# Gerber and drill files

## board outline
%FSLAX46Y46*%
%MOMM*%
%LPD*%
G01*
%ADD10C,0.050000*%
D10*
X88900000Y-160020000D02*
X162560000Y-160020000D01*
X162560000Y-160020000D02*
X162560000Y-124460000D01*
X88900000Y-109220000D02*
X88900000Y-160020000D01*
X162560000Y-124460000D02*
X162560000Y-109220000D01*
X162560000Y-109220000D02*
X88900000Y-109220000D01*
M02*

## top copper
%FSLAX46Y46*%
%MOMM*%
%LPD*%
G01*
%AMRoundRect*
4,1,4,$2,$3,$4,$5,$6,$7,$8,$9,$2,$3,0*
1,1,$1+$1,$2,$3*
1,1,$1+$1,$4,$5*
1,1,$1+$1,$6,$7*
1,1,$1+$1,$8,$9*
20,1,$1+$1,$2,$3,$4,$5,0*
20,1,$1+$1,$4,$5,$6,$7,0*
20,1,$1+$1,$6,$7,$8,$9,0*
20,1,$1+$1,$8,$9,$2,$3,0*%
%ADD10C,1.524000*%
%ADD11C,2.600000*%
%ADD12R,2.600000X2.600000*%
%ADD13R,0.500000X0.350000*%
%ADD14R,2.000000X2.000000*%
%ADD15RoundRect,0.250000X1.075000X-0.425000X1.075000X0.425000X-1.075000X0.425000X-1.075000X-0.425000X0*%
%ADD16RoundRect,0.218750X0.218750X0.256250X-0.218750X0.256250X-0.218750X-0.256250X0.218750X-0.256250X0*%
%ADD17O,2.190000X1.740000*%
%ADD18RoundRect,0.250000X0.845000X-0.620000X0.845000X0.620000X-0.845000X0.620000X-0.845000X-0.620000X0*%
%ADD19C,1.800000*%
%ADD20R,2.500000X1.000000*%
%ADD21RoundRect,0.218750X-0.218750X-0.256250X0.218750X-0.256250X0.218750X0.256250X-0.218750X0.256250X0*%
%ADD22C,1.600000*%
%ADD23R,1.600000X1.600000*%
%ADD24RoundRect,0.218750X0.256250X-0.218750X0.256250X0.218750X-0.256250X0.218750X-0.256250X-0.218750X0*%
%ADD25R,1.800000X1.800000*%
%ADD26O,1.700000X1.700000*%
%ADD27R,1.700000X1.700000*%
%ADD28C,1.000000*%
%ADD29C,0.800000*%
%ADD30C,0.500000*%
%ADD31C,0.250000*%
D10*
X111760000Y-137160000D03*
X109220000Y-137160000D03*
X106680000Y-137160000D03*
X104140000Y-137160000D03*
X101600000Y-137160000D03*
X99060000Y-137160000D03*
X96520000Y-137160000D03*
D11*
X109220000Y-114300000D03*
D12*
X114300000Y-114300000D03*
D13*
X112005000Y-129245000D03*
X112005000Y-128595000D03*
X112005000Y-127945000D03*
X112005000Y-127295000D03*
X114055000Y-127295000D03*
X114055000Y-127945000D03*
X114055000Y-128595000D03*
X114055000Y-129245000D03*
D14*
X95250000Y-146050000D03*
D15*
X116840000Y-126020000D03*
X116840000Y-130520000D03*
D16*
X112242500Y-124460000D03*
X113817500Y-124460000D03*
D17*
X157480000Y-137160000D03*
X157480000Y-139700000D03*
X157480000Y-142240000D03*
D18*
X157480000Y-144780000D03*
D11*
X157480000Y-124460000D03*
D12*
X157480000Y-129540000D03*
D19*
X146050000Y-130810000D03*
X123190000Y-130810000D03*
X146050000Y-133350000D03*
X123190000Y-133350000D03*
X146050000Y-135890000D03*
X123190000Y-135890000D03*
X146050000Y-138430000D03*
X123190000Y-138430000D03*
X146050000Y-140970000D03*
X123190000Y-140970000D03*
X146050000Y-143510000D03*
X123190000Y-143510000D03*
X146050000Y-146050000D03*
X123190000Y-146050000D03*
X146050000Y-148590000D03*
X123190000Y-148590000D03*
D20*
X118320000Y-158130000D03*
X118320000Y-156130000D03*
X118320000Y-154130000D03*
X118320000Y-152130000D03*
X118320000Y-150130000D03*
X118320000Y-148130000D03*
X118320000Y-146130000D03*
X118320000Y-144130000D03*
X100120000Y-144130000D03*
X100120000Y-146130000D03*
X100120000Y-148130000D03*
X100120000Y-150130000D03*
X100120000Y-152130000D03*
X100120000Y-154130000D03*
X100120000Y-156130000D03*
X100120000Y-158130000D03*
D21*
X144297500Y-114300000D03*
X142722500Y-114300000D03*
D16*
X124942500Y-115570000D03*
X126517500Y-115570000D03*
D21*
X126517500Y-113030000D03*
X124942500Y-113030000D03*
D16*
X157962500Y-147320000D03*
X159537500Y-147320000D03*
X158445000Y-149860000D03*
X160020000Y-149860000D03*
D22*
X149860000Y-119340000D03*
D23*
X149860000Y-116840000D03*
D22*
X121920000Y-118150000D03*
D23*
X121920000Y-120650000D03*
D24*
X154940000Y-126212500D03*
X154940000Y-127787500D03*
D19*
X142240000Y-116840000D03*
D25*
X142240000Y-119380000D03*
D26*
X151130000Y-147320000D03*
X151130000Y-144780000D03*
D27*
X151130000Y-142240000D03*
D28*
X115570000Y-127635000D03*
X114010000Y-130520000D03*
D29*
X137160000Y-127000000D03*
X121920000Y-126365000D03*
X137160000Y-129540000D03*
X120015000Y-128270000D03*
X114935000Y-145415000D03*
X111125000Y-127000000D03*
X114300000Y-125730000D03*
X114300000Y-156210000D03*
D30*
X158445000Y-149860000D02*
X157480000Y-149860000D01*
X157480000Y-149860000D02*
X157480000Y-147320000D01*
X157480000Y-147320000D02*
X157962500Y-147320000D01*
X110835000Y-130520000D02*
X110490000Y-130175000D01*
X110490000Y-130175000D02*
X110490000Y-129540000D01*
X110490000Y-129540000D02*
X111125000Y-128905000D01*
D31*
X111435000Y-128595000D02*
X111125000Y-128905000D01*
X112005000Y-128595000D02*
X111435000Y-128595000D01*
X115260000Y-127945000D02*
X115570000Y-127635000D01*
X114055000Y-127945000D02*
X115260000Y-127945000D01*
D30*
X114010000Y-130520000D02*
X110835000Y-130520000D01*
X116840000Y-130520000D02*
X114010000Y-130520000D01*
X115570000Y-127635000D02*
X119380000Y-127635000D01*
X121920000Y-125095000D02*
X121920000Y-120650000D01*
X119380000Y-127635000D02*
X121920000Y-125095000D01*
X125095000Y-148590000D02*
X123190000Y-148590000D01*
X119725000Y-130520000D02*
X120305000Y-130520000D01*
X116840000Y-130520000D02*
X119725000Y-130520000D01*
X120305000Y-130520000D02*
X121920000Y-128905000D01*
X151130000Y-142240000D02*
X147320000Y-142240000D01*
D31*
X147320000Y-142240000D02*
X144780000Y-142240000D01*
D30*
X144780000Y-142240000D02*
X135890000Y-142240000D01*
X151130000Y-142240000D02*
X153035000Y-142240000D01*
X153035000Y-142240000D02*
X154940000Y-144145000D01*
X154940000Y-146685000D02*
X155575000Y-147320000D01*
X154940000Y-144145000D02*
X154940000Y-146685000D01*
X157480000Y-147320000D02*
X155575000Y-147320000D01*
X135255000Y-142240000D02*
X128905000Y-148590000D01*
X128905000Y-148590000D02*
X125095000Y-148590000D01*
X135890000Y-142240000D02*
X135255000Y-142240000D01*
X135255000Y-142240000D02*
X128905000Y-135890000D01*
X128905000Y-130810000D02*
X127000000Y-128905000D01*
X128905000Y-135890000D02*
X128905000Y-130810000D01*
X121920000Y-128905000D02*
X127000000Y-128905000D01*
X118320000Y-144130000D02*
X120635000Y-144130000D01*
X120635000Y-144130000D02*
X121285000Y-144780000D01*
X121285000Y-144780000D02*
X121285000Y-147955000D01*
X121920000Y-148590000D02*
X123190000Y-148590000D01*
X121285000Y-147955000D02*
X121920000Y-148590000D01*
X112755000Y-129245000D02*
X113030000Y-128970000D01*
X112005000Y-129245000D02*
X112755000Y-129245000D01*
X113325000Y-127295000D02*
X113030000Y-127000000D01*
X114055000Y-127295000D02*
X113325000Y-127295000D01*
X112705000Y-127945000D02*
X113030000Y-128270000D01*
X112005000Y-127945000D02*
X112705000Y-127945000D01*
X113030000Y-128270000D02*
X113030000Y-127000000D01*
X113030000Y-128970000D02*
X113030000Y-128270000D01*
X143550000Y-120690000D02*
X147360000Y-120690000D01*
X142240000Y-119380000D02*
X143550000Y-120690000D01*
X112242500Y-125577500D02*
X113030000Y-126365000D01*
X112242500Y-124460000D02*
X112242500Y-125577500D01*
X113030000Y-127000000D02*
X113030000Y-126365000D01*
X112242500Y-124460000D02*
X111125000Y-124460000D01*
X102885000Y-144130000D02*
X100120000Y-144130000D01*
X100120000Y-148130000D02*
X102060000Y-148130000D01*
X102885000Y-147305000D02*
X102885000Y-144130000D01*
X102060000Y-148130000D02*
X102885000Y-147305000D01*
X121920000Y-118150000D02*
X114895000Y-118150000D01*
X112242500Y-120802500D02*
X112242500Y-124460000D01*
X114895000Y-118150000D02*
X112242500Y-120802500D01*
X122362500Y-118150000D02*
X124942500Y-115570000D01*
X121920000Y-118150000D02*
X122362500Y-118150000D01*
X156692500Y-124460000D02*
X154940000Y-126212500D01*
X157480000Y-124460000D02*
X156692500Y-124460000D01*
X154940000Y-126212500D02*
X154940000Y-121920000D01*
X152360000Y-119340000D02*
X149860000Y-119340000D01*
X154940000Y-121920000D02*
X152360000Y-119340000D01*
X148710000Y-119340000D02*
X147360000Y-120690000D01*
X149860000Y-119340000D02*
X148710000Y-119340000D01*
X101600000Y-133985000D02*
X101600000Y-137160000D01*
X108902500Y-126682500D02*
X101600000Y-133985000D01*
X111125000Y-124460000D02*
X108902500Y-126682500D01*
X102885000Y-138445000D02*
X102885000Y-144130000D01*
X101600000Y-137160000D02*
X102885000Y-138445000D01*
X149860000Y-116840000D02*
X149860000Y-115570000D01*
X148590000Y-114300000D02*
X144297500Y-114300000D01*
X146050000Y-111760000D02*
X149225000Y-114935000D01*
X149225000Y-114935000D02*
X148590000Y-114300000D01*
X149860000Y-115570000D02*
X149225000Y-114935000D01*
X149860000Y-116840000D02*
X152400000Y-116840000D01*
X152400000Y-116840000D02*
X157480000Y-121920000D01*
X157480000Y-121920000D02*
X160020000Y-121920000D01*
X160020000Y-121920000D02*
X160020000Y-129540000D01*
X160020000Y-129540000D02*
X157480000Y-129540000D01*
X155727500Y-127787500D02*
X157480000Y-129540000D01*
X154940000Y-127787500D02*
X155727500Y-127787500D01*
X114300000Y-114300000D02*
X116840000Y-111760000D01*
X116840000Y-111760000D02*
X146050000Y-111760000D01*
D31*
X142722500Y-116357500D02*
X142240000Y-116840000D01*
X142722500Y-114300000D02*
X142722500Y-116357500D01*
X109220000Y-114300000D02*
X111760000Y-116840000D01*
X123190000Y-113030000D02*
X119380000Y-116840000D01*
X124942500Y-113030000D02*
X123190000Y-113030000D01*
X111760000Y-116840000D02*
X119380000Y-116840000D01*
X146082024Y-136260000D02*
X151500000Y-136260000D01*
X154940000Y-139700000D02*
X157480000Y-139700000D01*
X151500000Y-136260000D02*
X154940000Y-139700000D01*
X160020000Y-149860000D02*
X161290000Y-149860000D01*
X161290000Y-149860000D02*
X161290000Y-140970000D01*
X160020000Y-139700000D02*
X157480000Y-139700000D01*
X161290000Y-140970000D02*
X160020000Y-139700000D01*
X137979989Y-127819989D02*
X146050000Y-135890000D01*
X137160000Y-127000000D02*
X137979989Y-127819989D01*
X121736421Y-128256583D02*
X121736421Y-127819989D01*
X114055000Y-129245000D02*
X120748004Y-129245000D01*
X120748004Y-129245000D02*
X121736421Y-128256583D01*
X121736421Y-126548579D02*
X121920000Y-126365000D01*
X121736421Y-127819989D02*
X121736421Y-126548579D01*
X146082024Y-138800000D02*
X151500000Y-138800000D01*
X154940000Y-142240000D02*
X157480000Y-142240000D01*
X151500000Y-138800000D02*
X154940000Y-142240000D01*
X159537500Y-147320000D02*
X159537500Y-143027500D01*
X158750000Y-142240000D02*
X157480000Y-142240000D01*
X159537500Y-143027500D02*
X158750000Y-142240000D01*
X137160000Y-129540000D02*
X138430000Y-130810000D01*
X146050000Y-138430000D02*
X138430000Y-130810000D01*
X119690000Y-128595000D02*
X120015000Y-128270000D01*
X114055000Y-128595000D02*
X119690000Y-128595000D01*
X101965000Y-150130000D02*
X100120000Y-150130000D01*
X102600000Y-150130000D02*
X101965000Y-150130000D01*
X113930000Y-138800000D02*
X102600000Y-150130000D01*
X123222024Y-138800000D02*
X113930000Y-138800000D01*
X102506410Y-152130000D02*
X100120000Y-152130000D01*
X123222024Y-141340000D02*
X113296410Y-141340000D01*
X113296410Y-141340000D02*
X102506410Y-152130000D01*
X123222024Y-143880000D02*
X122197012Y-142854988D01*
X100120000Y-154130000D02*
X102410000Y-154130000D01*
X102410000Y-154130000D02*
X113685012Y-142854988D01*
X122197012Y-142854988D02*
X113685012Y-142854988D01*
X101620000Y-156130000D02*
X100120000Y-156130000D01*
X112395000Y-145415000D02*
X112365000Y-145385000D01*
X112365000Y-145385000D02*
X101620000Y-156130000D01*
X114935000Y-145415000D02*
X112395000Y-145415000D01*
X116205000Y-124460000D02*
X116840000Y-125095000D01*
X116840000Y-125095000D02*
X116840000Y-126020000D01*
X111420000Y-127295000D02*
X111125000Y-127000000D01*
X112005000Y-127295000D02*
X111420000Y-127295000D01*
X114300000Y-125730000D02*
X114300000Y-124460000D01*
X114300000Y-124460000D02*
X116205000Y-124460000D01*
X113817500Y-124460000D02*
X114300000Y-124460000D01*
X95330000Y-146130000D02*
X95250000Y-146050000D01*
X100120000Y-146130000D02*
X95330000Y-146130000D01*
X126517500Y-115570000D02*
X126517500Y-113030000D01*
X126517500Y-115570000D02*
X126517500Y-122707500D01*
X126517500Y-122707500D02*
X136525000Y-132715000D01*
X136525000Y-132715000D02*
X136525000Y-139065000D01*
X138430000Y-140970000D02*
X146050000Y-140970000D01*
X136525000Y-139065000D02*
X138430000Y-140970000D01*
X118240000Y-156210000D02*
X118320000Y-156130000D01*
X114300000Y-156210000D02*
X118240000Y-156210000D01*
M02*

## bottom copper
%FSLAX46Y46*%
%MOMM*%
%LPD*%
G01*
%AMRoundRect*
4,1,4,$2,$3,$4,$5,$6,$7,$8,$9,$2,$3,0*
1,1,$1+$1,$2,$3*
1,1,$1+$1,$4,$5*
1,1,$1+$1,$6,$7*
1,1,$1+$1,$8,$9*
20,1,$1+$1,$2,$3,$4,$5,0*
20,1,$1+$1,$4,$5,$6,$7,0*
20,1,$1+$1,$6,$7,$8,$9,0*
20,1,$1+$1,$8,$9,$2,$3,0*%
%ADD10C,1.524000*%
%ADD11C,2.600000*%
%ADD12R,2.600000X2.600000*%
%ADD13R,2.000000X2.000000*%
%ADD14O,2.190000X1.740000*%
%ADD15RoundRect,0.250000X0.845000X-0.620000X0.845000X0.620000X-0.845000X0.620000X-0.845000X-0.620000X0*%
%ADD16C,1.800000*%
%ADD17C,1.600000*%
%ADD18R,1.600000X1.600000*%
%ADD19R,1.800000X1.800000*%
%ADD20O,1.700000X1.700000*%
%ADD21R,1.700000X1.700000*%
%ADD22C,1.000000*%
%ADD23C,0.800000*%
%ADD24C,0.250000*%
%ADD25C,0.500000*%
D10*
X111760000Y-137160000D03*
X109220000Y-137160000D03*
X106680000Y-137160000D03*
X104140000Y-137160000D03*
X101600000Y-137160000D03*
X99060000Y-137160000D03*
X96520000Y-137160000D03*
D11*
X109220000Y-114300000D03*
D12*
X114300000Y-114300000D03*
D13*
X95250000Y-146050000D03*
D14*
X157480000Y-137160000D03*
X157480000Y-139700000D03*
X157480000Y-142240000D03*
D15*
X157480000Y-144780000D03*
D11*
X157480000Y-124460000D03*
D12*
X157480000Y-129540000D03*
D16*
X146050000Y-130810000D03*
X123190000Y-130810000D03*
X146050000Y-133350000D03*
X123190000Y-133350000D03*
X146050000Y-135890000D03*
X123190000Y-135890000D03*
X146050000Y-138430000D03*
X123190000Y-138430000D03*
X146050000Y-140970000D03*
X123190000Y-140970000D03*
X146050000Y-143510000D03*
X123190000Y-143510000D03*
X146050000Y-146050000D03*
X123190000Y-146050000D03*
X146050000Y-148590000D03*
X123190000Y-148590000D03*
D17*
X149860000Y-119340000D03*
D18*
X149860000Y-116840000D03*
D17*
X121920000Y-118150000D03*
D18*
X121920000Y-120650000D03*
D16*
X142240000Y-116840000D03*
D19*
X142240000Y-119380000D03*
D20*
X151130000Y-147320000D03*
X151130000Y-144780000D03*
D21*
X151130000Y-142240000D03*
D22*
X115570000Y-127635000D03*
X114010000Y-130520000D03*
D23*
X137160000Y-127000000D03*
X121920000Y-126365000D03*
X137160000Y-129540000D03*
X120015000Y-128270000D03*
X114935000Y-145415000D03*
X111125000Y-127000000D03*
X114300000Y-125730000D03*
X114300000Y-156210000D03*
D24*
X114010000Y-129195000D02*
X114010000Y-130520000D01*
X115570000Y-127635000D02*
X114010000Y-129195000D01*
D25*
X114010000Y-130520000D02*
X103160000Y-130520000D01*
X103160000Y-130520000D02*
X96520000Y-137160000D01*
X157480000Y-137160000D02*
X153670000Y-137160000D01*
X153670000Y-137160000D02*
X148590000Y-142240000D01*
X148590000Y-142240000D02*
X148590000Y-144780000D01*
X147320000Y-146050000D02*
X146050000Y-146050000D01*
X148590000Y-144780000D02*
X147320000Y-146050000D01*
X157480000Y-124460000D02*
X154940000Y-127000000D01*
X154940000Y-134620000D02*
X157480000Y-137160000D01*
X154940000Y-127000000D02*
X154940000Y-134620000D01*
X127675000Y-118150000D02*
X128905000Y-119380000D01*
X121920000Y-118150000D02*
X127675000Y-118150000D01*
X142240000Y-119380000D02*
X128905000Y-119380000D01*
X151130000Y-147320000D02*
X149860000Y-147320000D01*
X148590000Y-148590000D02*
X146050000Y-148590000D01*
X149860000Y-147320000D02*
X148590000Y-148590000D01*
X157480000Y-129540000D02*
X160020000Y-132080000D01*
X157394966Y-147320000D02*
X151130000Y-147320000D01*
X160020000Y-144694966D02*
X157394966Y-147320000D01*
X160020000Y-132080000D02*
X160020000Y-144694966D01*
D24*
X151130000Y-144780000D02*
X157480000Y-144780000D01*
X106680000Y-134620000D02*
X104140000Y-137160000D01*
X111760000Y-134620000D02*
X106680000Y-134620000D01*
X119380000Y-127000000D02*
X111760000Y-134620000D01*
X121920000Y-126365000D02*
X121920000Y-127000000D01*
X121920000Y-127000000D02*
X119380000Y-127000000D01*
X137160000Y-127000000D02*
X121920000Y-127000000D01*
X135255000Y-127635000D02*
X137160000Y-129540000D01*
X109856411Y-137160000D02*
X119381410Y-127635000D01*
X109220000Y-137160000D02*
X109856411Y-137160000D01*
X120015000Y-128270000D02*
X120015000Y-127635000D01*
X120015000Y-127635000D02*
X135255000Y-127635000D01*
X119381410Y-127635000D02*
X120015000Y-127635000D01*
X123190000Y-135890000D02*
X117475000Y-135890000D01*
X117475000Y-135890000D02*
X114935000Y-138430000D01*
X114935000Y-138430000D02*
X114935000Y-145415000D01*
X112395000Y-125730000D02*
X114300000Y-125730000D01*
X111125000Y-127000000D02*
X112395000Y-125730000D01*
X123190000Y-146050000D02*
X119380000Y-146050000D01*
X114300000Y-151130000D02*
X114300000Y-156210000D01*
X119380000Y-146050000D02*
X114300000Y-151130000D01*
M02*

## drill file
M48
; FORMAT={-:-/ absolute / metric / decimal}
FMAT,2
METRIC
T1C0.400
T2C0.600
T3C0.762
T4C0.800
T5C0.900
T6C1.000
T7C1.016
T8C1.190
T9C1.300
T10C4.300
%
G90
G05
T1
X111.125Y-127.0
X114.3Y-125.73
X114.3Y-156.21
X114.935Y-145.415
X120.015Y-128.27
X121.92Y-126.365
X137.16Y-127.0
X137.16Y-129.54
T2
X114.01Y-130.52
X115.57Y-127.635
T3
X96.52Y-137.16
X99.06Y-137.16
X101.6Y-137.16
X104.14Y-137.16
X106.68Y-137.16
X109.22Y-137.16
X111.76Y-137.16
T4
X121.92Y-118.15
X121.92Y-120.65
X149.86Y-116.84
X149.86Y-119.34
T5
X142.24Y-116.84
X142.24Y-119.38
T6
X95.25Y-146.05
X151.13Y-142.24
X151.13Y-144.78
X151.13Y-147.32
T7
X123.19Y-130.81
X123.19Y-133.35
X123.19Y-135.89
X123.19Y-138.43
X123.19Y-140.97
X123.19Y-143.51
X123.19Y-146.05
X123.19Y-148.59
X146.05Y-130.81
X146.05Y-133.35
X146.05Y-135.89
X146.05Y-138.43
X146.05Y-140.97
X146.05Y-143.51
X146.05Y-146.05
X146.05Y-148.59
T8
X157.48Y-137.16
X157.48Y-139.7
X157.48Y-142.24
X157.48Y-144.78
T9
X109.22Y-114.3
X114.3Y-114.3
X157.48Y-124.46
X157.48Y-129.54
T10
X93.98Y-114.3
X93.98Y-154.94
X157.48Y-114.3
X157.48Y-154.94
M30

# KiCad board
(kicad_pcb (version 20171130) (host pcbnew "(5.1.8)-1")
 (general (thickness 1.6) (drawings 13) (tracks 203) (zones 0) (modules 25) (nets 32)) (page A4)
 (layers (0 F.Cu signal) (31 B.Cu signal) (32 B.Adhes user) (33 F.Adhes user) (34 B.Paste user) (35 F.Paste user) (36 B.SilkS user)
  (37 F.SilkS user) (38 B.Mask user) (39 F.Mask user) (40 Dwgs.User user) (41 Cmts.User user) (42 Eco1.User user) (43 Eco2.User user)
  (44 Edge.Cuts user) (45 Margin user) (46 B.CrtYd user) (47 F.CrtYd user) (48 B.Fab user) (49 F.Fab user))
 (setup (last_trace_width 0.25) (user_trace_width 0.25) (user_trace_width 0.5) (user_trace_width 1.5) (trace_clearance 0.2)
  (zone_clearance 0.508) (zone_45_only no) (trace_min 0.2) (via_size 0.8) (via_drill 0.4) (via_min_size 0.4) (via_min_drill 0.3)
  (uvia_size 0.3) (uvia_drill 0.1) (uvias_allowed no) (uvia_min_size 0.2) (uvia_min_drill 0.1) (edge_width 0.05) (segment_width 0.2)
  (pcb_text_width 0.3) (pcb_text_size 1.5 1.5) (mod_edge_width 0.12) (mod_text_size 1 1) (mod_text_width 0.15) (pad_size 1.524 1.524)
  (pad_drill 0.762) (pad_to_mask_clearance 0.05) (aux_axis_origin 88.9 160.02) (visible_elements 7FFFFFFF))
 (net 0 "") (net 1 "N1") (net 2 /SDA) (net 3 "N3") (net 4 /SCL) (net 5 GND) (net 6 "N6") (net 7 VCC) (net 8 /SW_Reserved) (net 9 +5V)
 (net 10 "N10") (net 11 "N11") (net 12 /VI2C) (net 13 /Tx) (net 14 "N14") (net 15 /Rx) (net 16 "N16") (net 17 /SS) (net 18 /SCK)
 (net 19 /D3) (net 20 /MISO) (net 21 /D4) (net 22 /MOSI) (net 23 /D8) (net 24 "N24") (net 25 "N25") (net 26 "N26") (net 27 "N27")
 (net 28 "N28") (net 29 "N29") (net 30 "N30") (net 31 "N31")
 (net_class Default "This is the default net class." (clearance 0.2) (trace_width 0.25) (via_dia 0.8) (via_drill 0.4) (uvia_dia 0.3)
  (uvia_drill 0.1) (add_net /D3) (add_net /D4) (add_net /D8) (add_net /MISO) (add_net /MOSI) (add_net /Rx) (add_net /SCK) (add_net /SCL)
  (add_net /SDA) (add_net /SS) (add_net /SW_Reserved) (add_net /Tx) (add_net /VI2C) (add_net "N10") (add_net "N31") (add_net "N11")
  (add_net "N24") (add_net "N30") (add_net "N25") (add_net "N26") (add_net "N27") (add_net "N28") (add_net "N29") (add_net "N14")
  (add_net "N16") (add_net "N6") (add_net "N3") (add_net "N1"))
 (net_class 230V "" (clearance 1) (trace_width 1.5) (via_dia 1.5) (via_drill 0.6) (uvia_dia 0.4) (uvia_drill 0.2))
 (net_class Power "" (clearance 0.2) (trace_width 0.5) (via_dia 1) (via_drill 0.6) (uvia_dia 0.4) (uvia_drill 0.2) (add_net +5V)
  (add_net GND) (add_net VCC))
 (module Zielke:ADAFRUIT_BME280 (layer F.Cu) (at 104.14 137.16 90)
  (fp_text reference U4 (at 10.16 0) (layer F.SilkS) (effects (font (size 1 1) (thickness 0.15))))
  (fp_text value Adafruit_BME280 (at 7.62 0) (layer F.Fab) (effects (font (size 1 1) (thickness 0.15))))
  (pad 7 thru_hole circle (at 0 7.62 90) (size 1.524 1.524) (drill 0.762) (layers *.Cu *.Mask) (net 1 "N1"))
  (pad 6 thru_hole circle (at 0 5.08 90) (size 1.524 1.524) (drill 0.762) (layers *.Cu *.Mask) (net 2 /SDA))
  (pad 5 thru_hole circle (at 0 2.54 90) (size 1.524 1.524) (drill 0.762) (layers *.Cu *.Mask) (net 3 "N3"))
  (pad 4 thru_hole circle (at 0 0 90) (size 1.524 1.524) (drill 0.762) (layers *.Cu *.Mask) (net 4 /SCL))
  (pad 3 thru_hole circle (at 0 -2.54 90) (size 1.524 1.524) (drill 0.762) (layers *.Cu *.Mask) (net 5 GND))
  (pad 2 thru_hole circle (at 0 -5.08 90) (size 1.524 1.524) (drill 0.762) (layers *.Cu *.Mask) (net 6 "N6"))
  (pad 1 thru_hole circle (at 0 -7.62 90) (size 1.524 1.524) (drill 0.762) (layers *.Cu *.Mask) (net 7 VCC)))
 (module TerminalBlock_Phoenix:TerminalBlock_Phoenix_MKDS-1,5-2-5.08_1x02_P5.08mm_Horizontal (layer F.Cu) (at 114.3 114.3 180)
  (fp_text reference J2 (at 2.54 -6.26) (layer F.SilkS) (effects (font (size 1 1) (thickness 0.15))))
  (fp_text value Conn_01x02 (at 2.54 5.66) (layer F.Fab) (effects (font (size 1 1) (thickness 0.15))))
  (pad 2 thru_hole circle (at 5.08 0 180) (size 2.6 2.6) (drill 1.3) (layers *.Cu *.Mask) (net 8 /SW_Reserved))
  (pad 1 thru_hole rect (at 0 0 180) (size 2.6 2.6) (drill 1.3) (layers *.Cu *.Mask) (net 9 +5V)))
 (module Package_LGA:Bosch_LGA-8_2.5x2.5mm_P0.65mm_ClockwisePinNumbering (layer F.Cu) (at 113.03 128.27 270)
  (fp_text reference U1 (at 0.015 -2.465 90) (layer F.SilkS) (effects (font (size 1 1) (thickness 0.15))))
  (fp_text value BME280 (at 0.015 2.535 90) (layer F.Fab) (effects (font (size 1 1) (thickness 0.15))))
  (pad 5 smd rect (at 0.975 1.025) (size 0.5 0.35) (layers F.Cu F.Paste F.Mask) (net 5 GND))
  (pad 6 smd rect (at 0.325 1.025) (size 0.5 0.35) (layers F.Cu F.Paste F.Mask) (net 7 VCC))
  (pad 7 smd rect (at -0.325 1.025) (size 0.5 0.35) (layers F.Cu F.Paste F.Mask) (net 5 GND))
  (pad 8 smd rect (at -0.975 1.025) (size 0.5 0.35) (layers F.Cu F.Paste F.Mask) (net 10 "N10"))
  (pad 1 smd rect (at -0.975 -1.025) (size 0.5 0.35) (layers F.Cu F.Paste F.Mask) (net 5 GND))
  (pad 2 smd rect (at -0.325 -1.025) (size 0.5 0.35) (layers F.Cu F.Paste F.Mask) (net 7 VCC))
  (pad 3 smd rect (at 0.325 -1.025) (size 0.5 0.35) (layers F.Cu F.Paste F.Mask) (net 2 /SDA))
  (pad 4 smd rect (at 0.975 -1.025) (size 0.5 0.35) (layers F.Cu F.Paste F.Mask) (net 4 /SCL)))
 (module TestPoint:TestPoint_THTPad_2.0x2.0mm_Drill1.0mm (layer F.Cu) (at 95.25 146.05)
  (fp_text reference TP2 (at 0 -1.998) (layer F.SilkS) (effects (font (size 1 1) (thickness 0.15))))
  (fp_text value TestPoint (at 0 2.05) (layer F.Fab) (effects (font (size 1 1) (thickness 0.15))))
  (pad 1 thru_hole rect (at 0 0) (size 2 2) (drill 1) (layers *.Cu *.Mask) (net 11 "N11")))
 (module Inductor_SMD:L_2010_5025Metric (layer F.Cu) (at 116.84 128.27 90)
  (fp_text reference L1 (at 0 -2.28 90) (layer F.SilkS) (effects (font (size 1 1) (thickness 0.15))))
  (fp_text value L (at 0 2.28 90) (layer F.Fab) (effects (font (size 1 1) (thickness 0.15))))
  (pad 2 smd roundrect (at 2.25 0 90) (size 1.35 2.65) (layers F.Cu F.Paste F.Mask) (roundrect_rratio 0.185185) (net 10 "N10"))
  (pad 1 smd roundrect (at -2.25 0 90) (size 1.35 2.65) (layers F.Cu F.Paste F.Mask) (roundrect_rratio 0.185185) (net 7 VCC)))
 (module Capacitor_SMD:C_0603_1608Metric (layer F.Cu) (at 113.03 124.46 180)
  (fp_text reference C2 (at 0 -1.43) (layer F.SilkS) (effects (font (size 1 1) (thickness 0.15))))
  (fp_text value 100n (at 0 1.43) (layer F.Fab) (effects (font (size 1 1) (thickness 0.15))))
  (pad 2 smd roundrect (at 0.7875 0 180) (size 0.875 0.95) (layers F.Cu F.Paste F.Mask) (roundrect_rratio 0.25) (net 5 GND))
  (pad 1 smd roundrect (at -0.7875 0 180) (size 0.875 0.95) (layers F.Cu F.Paste F.Mask) (roundrect_rratio 0.25) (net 10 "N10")))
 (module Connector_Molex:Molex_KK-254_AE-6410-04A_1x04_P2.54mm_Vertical (layer F.Cu) (at 157.48 144.78 90)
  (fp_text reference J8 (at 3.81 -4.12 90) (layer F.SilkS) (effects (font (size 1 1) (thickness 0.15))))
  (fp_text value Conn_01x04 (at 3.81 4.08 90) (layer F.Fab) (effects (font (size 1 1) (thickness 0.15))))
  (pad 4 thru_hole oval (at 7.62 0 90) (size 1.74 2.19) (drill 1.19) (layers *.Cu *.Mask) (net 5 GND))
  (pad 3 thru_hole oval (at 5.08 0 90) (size 1.74 2.19) (drill 1.19) (layers *.Cu *.Mask) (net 4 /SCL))
  (pad 2 thru_hole oval (at 2.54 0 90) (size 1.74 2.19) (drill 1.19) (layers *.Cu *.Mask) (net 2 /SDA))
  (pad 1 thru_hole roundrect (at 0 0 90) (size 1.74 2.19) (drill 1.19) (layers *.Cu *.Mask) (roundrect_rratio 0.143678) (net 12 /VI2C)))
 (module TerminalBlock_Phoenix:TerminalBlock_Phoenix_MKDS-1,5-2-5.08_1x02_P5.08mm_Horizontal (layer F.Cu) (at 157.48 129.54 90)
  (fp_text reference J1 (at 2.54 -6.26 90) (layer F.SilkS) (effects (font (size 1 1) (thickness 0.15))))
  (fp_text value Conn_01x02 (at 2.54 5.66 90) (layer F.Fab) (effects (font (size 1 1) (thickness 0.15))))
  (pad 2 thru_hole circle (at 5.08 0 90) (size 2.6 2.6) (drill 1.3) (layers *.Cu *.Mask) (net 5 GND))
  (pad 1 thru_hole rect (at 0 0 90) (size 2.6 2.6) (drill 1.3) (layers *.Cu *.Mask) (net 9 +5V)))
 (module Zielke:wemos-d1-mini (layer F.Cu) (at 134.62 139.7 90)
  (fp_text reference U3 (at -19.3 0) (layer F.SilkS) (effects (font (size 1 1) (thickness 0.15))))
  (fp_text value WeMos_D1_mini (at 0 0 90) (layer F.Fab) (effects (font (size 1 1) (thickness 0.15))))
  (pad 16 thru_hole circle (at 8.89 11.43 90) (size 1.8 1.8) (drill 1.016) (layers *.Cu *.Mask) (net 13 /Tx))
  (pad 1 thru_hole circle (at 8.89 -11.43 90) (size 1.8 1.8) (drill 1.016) (layers *.Cu *.Mask) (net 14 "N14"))
  (pad 15 thru_hole circle (at 6.35 11.43 90) (size 1.8 1.8) (drill 1.016) (layers *.Cu *.Mask) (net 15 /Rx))
  (pad 2 thru_hole circle (at 6.35 -11.43 90) (size 1.8 1.8) (drill 1.016) (layers *.Cu *.Mask) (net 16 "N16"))
  (pad 14 thru_hole circle (at 3.81 11.43 90) (size 1.8 1.8) (drill 1.016) (layers *.Cu *.Mask) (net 4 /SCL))
  (pad 3 thru_hole circle (at 3.81 -11.43 90) (size 1.8 1.8) (drill 1.016) (layers *.Cu *.Mask) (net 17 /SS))
  (pad 13 thru_hole circle (at 1.27 11.43 90) (size 1.8 1.8) (drill 1.016) (layers *.Cu *.Mask) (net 2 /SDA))
  (pad 4 thru_hole circle (at 1.27 -11.43 90) (size 1.8 1.8) (drill 1.016) (layers *.Cu *.Mask) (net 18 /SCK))
  (pad 12 thru_hole circle (at -1.27 11.43 90) (size 1.8 1.8) (drill 1.016) (layers *.Cu *.Mask) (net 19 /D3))
  (pad 5 thru_hole circle (at -1.27 -11.43 90) (size 1.8 1.8) (drill 1.016) (layers *.Cu *.Mask) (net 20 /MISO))
  (pad 11 thru_hole circle (at -3.81 11.43 90) (size 1.8 1.8) (drill 1.016) (layers *.Cu *.Mask) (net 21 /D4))
  (pad 6 thru_hole circle (at -3.81 -11.43 180) (size 1.8 1.8) (drill 1.016) (layers *.Cu *.Mask) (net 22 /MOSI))
  (pad 10 thru_hole circle (at -6.35 11.43 90) (size 1.8 1.8) (drill 1.016) (layers *.Cu *.Mask) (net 5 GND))
  (pad 7 thru_hole circle (at -6.35 -11.43 90) (size 1.8 1.8) (drill 1.016) (layers *.Cu *.Mask) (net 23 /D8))
  (pad 9 thru_hole circle (at -8.89 11.43 90) (size 1.8 1.8) (drill 1.016) (layers *.Cu *.Mask) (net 9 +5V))
  (pad 8 thru_hole circle (at -8.89 -11.43 90) (size 1.8 1.8) (drill 1.016) (layers *.Cu *.Mask) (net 7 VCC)))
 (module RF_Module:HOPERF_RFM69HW (layer F.Cu) (at 109.22 151.13 180)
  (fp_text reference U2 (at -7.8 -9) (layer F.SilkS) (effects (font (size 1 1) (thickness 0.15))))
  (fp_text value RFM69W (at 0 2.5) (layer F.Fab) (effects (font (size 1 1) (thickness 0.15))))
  (pad 1 smd rect (at -9.1 -7 180) (size 2.5 1) (layers F.Cu F.Paste F.Mask) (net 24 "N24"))
  (pad 2 smd rect (at -9.1 -5 180) (size 2.5 1) (layers F.Cu F.Paste F.Mask) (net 23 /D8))
  (pad 3 smd rect (at -9.1 -3 180) (size 2.5 1) (layers F.Cu F.Paste F.Mask) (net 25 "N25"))
  (pad 4 smd rect (at -9.1 -1 180) (size 2.5 1) (layers F.Cu F.Paste F.Mask) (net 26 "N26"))
  (pad 5 smd rect (at -9.1 1 180) (size 2.5 1) (layers F.Cu F.Paste F.Mask) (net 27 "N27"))
  (pad 6 smd rect (at -9.1 3 180) (size 2.5 1) (layers F.Cu F.Paste F.Mask) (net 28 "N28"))
  (pad 7 smd rect (at -9.1 5 180) (size 2.5 1) (layers F.Cu F.Paste F.Mask) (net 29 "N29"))
  (pad 8 smd rect (at -9.1 7 180) (size 2.5 1) (layers F.Cu F.Paste F.Mask) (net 7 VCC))
  (pad 9 smd rect (at 9.1 7 180) (size 2.5 1) (layers F.Cu F.Paste F.Mask) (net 5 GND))
  (pad 10 smd rect (at 9.1 5 180) (size 2.5 1) (layers F.Cu F.Paste F.Mask) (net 11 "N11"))
  (pad 11 smd rect (at 9.1 3 180) (size 2.5 1) (layers F.Cu F.Paste F.Mask) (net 5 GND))
  (pad 12 smd rect (at 9.1 1 180) (size 2.5 1) (layers F.Cu F.Paste F.Mask) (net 18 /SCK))
  (pad 13 smd rect (at 9.1 -1 180) (size 2.5 1) (layers F.Cu F.Paste F.Mask) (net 20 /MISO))
  (pad 14 smd rect (at 9.1 -3 180) (size 2.5 1) (layers F.Cu F.Paste F.Mask) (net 22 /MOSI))
  (pad 15 smd rect (at 9.1 -5 180) (size 2.5 1) (layers F.Cu F.Paste F.Mask) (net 17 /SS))
  (pad 16 smd rect (at 9.1 -7 180) (size 2.5 1) (layers F.Cu F.Paste F.Mask) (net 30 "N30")))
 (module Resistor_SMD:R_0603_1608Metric (layer F.Cu) (at 143.51 114.3)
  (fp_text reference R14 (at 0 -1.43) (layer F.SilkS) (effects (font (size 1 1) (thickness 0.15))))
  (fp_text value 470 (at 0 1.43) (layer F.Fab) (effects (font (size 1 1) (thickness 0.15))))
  (pad 2 smd roundrect (at 0.7875 0) (size 0.875 0.95) (layers F.Cu F.Paste F.Mask) (roundrect_rratio 0.25) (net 9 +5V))
  (pad 1 smd roundrect (at -0.7875 0) (size 0.875 0.95) (layers F.Cu F.Paste F.Mask) (roundrect_rratio 0.25) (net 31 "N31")))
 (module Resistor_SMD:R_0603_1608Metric (layer F.Cu) (at 125.73 115.57 180)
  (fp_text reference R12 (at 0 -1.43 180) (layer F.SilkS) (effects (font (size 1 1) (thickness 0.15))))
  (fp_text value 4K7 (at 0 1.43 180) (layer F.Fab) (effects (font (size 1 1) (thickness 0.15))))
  (pad 2 smd roundrect (at 0.7875 0 180) (size 0.875 0.95) (layers F.Cu F.Paste F.Mask) (roundrect_rratio 0.25) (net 5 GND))
  (pad 1 smd roundrect (at -0.7875 0 180) (size 0.875 0.95) (layers F.Cu F.Paste F.Mask) (roundrect_rratio 0.25) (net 19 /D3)))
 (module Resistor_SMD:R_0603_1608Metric (layer F.Cu) (at 125.73 113.03)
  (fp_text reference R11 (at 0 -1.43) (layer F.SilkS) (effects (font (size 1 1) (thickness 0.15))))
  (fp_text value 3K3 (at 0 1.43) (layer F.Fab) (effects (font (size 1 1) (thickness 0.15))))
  (pad 2 smd roundrect (at 0.7875 0) (size 0.875 0.95) (layers F.Cu F.Paste F.Mask) (roundrect_rratio 0.25) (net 19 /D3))
  (pad 1 smd roundrect (at -0.7875 0) (size 0.875 0.95) (layers F.Cu F.Paste F.Mask) (roundrect_rratio 0.25) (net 8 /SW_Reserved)))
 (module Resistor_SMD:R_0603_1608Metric (layer F.Cu) (at 158.75 147.32 180)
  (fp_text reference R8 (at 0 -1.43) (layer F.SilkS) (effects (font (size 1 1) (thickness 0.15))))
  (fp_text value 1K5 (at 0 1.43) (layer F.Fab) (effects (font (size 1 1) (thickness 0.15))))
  (pad 2 smd roundrect (at 0.7875 0 180) (size 0.875 0.95) (layers F.Cu F.Paste F.Mask) (roundrect_rratio 0.25) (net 7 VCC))
  (pad 1 smd roundrect (at -0.7875 0 180) (size 0.875 0.95) (layers F.Cu F.Paste F.Mask) (roundrect_rratio 0.25) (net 2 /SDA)))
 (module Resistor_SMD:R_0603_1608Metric (layer F.Cu) (at 159.2325 149.86 180)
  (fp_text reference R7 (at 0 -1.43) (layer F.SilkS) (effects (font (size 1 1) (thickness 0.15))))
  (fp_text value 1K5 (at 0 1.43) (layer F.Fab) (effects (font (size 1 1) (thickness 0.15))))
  (pad 2 smd roundrect (at 0.7875 0 180) (size 0.875 0.95) (layers F.Cu F.Paste F.Mask) (roundrect_rratio 0.25) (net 7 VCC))
  (pad 1 smd roundrect (at -0.7875 0 180) (size 0.875 0.95) (layers F.Cu F.Paste F.Mask) (roundrect_rratio 0.25) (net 4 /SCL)))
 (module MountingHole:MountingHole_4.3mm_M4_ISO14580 (layer F.Cu) (at 157.48 114.3)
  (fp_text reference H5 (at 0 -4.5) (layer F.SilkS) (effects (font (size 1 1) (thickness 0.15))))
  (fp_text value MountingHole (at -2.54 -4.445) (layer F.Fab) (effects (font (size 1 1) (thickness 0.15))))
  (pad 1 np_thru_hole circle (at 0 0) (size 4.3 4.3) (drill 4.3) (layers *.Cu *.Mask)))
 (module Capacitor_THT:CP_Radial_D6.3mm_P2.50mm (layer F.Cu) (at 149.86 116.84 270)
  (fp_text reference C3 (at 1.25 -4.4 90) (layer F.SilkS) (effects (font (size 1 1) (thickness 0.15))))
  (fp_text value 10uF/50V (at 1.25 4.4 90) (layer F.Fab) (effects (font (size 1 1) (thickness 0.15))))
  (pad 2 thru_hole circle (at 2.5 0 270) (size 1.6 1.6) (drill 0.8) (layers *.Cu *.Mask) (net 5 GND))
  (pad 1 thru_hole rect (at 0 0 270) (size 1.6 1.6) (drill 0.8) (layers *.Cu *.Mask) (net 9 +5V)))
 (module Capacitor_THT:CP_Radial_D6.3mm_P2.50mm (layer F.Cu) (at 121.92 120.65 90)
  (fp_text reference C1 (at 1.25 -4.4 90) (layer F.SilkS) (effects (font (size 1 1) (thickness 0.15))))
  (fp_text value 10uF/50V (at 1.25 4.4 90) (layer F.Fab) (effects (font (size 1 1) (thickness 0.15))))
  (pad 2 thru_hole circle (at 2.5 0 90) (size 1.6 1.6) (drill 0.8) (layers *.Cu *.Mask) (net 5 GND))
  (pad 1 thru_hole rect (at 0 0 90) (size 1.6 1.6) (drill 0.8) (layers *.Cu *.Mask) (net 7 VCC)))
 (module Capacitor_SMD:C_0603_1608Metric (layer F.Cu) (at 154.94 127 90)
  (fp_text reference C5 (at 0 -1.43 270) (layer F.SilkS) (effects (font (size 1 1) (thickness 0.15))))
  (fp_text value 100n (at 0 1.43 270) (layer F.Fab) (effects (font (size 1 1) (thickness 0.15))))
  (pad 2 smd roundrect (at 0.7875 0 90) (size 0.875 0.95) (layers F.Cu F.Paste F.Mask) (roundrect_rratio 0.25) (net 5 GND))
  (pad 1 smd roundrect (at -0.7875 0 90) (size 0.875 0.95) (layers F.Cu F.Paste F.Mask) (roundrect_rratio 0.25) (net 9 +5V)))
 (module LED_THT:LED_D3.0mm (layer F.Cu) (at 142.24 119.38 90)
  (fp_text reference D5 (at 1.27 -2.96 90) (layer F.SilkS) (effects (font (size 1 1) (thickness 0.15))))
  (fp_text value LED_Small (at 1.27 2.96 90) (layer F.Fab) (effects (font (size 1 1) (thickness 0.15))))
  (pad 2 thru_hole circle (at 2.54 0 90) (size 1.8 1.8) (drill 0.9) (layers *.Cu *.Mask) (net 31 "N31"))
  (pad 1 thru_hole rect (at 0 0 90) (size 1.8 1.8) (drill 0.9) (layers *.Cu *.Mask) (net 5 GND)))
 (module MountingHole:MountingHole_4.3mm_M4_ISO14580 (layer F.Cu) (at 93.98 114.3)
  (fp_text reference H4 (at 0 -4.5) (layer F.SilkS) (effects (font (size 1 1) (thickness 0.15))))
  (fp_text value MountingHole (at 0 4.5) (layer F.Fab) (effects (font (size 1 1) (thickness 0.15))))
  (pad 1 np_thru_hole circle (at 0 0) (size 4.3 4.3) (drill 4.3) (layers *.Cu *.Mask)))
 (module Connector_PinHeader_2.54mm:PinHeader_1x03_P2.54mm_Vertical (layer F.Cu) (at 151.13 142.24)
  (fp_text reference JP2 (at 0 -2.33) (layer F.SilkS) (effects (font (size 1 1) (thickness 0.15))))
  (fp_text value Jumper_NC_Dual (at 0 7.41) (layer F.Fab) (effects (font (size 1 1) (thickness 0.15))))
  (pad 3 thru_hole oval (at 0 5.08) (size 1.7 1.7) (drill 1) (layers *.Cu *.Mask) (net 9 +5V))
  (pad 2 thru_hole oval (at 0 2.54) (size 1.7 1.7) (drill 1) (layers *.Cu *.Mask) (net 12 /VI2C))
  (pad 1 thru_hole rect (at 0 0) (size 1.7 1.7) (drill 1) (layers *.Cu *.Mask) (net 7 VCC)))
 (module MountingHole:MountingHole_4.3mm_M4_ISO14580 (layer F.Cu) (at 93.98 154.94)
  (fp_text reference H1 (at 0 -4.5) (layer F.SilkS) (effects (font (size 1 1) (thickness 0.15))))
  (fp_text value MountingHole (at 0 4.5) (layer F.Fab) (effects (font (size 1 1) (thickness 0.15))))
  (pad 1 np_thru_hole circle (at 0 0) (size 4.3 4.3) (drill 4.3) (layers *.Cu *.Mask)))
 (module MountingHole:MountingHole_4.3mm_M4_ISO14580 (layer F.Cu) (at 157.48 154.94)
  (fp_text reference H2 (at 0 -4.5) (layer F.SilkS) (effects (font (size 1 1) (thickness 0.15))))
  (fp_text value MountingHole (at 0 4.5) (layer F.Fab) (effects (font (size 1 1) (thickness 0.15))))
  (pad 1 np_thru_hole circle (at 0 0) (size 4.3 4.3) (drill 4.3) (layers *.Cu *.Mask)))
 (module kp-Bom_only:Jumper (layer F.Cu) (at 151.13 146.05)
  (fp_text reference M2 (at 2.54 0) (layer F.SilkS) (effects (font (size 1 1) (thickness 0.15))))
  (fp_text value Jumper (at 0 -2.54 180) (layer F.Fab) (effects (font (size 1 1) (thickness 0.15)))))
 (gr_line (start 88.9 160.02) (end 162.56 160.02) (layer Edge.Cuts) (width 0.05))
 (gr_line (start 162.56 160.02) (end 162.56 124.46) (layer Edge.Cuts) (width 0.05))
 (gr_line (start 88.9 109.22) (end 88.9 160.02) (layer Edge.Cuts) (width 0.05))
 (gr_line (start 162.56 124.46) (end 162.56 109.22) (layer Edge.Cuts) (width 0.05))
 (gr_line (start 162.56 109.22) (end 88.9 109.22) (layer Edge.Cuts) (width 0.05))
 (segment (start 158.445 149.86) (end 157.48 149.86) (width 0.5) (layer F.Cu) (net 7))
 (segment (start 157.48 149.86) (end 157.48 147.32) (width 0.5) (layer F.Cu) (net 7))
 (segment (start 157.48 147.32) (end 157.9625 147.32) (width 0.5) (layer F.Cu) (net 7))
 (segment (start 110.835 130.52) (end 110.49 130.175) (width 0.5) (layer F.Cu) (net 7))
 (segment (start 110.49 130.175) (end 110.49 129.54) (width 0.5) (layer F.Cu) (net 7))
 (segment (start 110.49 129.54) (end 111.125 128.905) (width 0.5) (layer F.Cu) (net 7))
 (segment (start 111.435 128.595) (end 111.125 128.905) (width 0.25) (layer F.Cu) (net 7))
 (segment (start 112.005 128.595) (end 111.435 128.595) (width 0.25) (layer F.Cu) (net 7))
 (via (at 115.57 127.635) (size 1) (drill 0.6) (layers F.Cu B.Cu) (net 7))
 (segment (start 115.26 127.945) (end 115.57 127.635) (width 0.25) (layer F.Cu) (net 7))
 (segment (start 114.055 127.945) (end 115.26 127.945) (width 0.25) (layer F.Cu) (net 7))
 (segment (start 114.01 129.195) (end 114.01 130.52) (width 0.25) (layer B.Cu) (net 7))
 (via (at 114.01 130.52) (size 1) (drill 0.6) (layers F.Cu B.Cu) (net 7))
 (segment (start 115.57 127.635) (end 114.01 129.195) (width 0.25) (layer B.Cu) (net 7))
 (segment (start 114.01 130.52) (end 110.835 130.52) (width 0.5) (layer F.Cu) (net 7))
 (segment (start 116.84 130.52) (end 114.01 130.52) (width 0.5) (layer F.Cu) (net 7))
 (segment (start 115.57 127.635) (end 119.38 127.635) (width 0.5) (layer F.Cu) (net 7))
 (segment (start 121.92 125.095) (end 121.92 120.65) (width 0.5) (layer F.Cu) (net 7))
 (segment (start 119.38 127.635) (end 121.92 125.095) (width 0.5) (layer F.Cu) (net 7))
 (segment (start 125.095 148.59) (end 123.19 148.59) (width 0.5) (layer F.Cu) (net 7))
 (segment (start 119.725 130.52) (end 120.305 130.52) (width 0.5) (layer F.Cu) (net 7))
 (segment (start 116.84 130.52) (end 119.725 130.52) (width 0.5) (layer F.Cu) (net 7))
 (segment (start 120.305 130.52) (end 121.92 128.905) (width 0.5) (layer F.Cu) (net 7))
 (segment (start 151.13 142.24) (end 147.32 142.24) (width 0.5) (layer F.Cu) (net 7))
 (segment (start 147.32 142.24) (end 144.78 142.24) (width 0.25) (layer F.Cu) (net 7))
 (segment (start 144.78 142.24) (end 135.89 142.24) (width 0.5) (layer F.Cu) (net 7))
 (segment (start 151.13 142.24) (end 153.035 142.24) (width 0.5) (layer F.Cu) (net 7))
 (segment (start 153.035 142.24) (end 154.94 144.145) (width 0.5) (layer F.Cu) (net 7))
 (segment (start 154.94 146.685) (end 155.575 147.32) (width 0.5) (layer F.Cu) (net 7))
 (segment (start 154.94 144.145) (end 154.94 146.685) (width 0.5) (layer F.Cu) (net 7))
 (segment (start 157.48 147.32) (end 155.575 147.32) (width 0.5) (layer F.Cu) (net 7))
 (segment (start 135.255 142.24) (end 128.905 148.59) (width 0.5) (layer F.Cu) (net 7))
 (segment (start 128.905 148.59) (end 125.095 148.59) (width 0.5) (layer F.Cu) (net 7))
 (segment (start 135.89 142.24) (end 135.255 142.24) (width 0.5) (layer F.Cu) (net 7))
 (segment (start 135.255 142.24) (end 128.905 135.89) (width 0.5) (layer F.Cu) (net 7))
 (segment (start 128.905 130.81) (end 127 128.905) (width 0.5) (layer F.Cu) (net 7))
 (segment (start 128.905 135.89) (end 128.905 130.81) (width 0.5) (layer F.Cu) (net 7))
 (segment (start 121.92 128.905) (end 127 128.905) (width 0.5) (layer F.Cu) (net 7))
 (segment (start 114.01 130.52) (end 103.16 130.52) (width 0.5) (layer B.Cu) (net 7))
 (segment (start 103.16 130.52) (end 96.52 137.16) (width 0.5) (layer B.Cu) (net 7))
 (segment (start 118.32 144.13) (end 120.635 144.13) (width 0.5) (layer F.Cu) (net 7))
 (segment (start 120.635 144.13) (end 121.285 144.78) (width 0.5) (layer F.Cu) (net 7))
 (segment (start 121.285 144.78) (end 121.285 147.955) (width 0.5) (layer F.Cu) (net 7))
 (segment (start 121.92 148.59) (end 123.19 148.59) (width 0.5) (layer F.Cu) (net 7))
 (segment (start 121.285 147.955) (end 121.92 148.59) (width 0.5) (layer F.Cu) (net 7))
 (segment (start 112.755 129.245) (end 113.03 128.97) (width 0.5) (layer F.Cu) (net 5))
 (segment (start 112.005 129.245) (end 112.755 129.245) (width 0.5) (layer F.Cu) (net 5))
 (segment (start 113.325 127.295) (end 113.03 127) (width 0.5) (layer F.Cu) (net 5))
 (segment (start 114.055 127.295) (end 113.325 127.295) (width 0.5) (layer F.Cu) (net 5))
 (segment (start 112.705 127.945) (end 113.03 128.27) (width 0.5) (layer F.Cu) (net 5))
 (segment (start 112.005 127.945) (end 112.705 127.945) (width 0.5) (layer F.Cu) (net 5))
 (segment (start 113.03 128.27) (end 113.03 127) (width 0.5) (layer F.Cu) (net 5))
 (segment (start 113.03 128.97) (end 113.03 128.27) (width 0.5) (layer F.Cu) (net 5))
 (segment (start 143.55 120.69) (end 147.36 120.69) (width 0.5) (layer F.Cu) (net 5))
 (segment (start 142.24 119.38) (end 143.55 120.69) (width 0.5) (layer F.Cu) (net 5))
 (segment (start 157.48 137.16) (end 153.67 137.16) (width 0.5) (layer B.Cu) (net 5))
 (segment (start 153.67 137.16) (end 148.59 142.24) (width 0.5) (layer B.Cu) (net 5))
 (segment (start 148.59 142.24) (end 148.59 144.78) (width 0.5) (layer B.Cu) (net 5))
 (segment (start 147.32 146.05) (end 146.05 146.05) (width 0.5) (layer B.Cu) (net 5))
 (segment (start 148.59 144.78) (end 147.32 146.05) (width 0.5) (layer B.Cu) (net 5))
 (segment (start 112.2425 125.5775) (end 113.03 126.365) (width 0.5) (layer F.Cu) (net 5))
 (segment (start 112.2425 124.46) (end 112.2425 125.5775) (width 0.5) (layer F.Cu) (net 5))
 (segment (start 113.03 127) (end 113.03 126.365) (width 0.5) (layer F.Cu) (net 5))
 (segment (start 112.2425 124.46) (end 111.125 124.46) (width 0.5) (layer F.Cu) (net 5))
 (segment (start 102.885 144.13) (end 100.12 144.13) (width 0.5) (layer F.Cu) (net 5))
 (segment (start 100.12 148.13) (end 102.06 148.13) (width 0.5) (layer F.Cu) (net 5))
 (segment (start 102.885 147.305) (end 102.885 144.13) (width 0.5) (layer F.Cu) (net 5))
 (segment (start 102.06 148.13) (end 102.885 147.305) (width 0.5) (layer F.Cu) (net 5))
 (segment (start 121.92 118.15) (end 114.895 118.15) (width 0.5) (layer F.Cu) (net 5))
 (segment (start 112.2425 120.8025) (end 112.2425 124.46) (width 0.5) (layer F.Cu) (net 5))
 (segment (start 114.895 118.15) (end 112.2425 120.8025) (width 0.5) (layer F.Cu) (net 5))
 (segment (start 122.3625 118.15) (end 124.9425 115.57) (width 0.5) (layer F.Cu) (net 5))
 (segment (start 121.92 118.15) (end 122.3625 118.15) (width 0.5) (layer F.Cu) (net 5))
 (segment (start 156.6925 124.46) (end 154.94 126.2125) (width 0.5) (layer F.Cu) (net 5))
 (segment (start 157.48 124.46) (end 156.6925 124.46) (width 0.5) (layer F.Cu) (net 5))
 (segment (start 154.94 126.2125) (end 154.94 121.92) (width 0.5) (layer F.Cu) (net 5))
 (segment (start 152.36 119.34) (end 149.86 119.34) (width 0.5) (layer F.Cu) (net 5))
 (segment (start 154.94 121.92) (end 152.36 119.34) (width 0.5) (layer F.Cu) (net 5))
 (segment (start 148.71 119.34) (end 147.36 120.69) (width 0.5) (layer F.Cu) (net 5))
 (segment (start 149.86 119.34) (end 148.71 119.34) (width 0.5) (layer F.Cu) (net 5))
 (segment (start 157.48 124.46) (end 154.94 127) (width 0.5) (layer B.Cu) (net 5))
 (segment (start 154.94 134.62) (end 157.48 137.16) (width 0.5) (layer B.Cu) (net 5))
 (segment (start 154.94 127) (end 154.94 134.62) (width 0.5) (layer B.Cu) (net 5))
 (segment (start 101.6 133.985) (end 101.6 137.16) (width 0.5) (layer F.Cu) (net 5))
 (segment (start 108.9025 126.6825) (end 101.6 133.985) (width 0.5) (layer F.Cu) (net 5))
 (segment (start 111.125 124.46) (end 108.9025 126.6825) (width 0.5) (layer F.Cu) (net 5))
 (segment (start 102.885 138.445) (end 102.885 144.13) (width 0.5) (layer F.Cu) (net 5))
 (segment (start 101.6 137.16) (end 102.885 138.445) (width 0.5) (layer F.Cu) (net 5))
 (segment (start 127.675 118.15) (end 128.905 119.38) (width 0.5) (layer B.Cu) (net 5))
 (segment (start 121.92 118.15) (end 127.675 118.15) (width 0.5) (layer B.Cu) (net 5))
 (segment (start 142.24 119.38) (end 128.905 119.38) (width 0.5) (layer B.Cu) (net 5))
 (segment (start 149.86 116.84) (end 149.86 115.57) (width 0.5) (layer F.Cu) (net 9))
 (segment (start 148.59 114.3) (end 144.2975 114.3) (width 0.5) (layer F.Cu) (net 9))
 (segment (start 151.13 147.32) (end 149.86 147.32) (width 0.5) (layer B.Cu) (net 9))
 (segment (start 148.59 148.59) (end 146.05 148.59) (width 0.5) (layer B.Cu) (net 9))
 (segment (start 149.86 147.32) (end 148.59 148.59) (width 0.5) (layer B.Cu) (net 9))
 (segment (start 146.05 111.76) (end 149.225 114.935) (width 0.5) (layer F.Cu) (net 9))
 (segment (start 149.225 114.935) (end 148.59 114.3) (width 0.5) (layer F.Cu) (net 9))
 (segment (start 149.86 115.57) (end 149.225 114.935) (width 0.5) (layer F.Cu) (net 9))
 (segment (start 149.86 116.84) (end 152.4 116.84) (width 0.5) (layer F.Cu) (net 9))
 (segment (start 152.4 116.84) (end 157.48 121.92) (width 0.5) (layer F.Cu) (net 9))
 (segment (start 157.48 121.92) (end 160.02 121.92) (width 0.5) (layer F.Cu) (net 9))
 (segment (start 160.02 121.92) (end 160.02 129.54) (width 0.5) (layer F.Cu) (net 9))
 (segment (start 160.02 129.54) (end 157.48 129.54) (width 0.5) (layer F.Cu) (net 9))
 (segment (start 155.7275 127.7875) (end 157.48 129.54) (width 0.5) (layer F.Cu) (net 9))
 (segment (start 154.94 127.7875) (end 155.7275 127.7875) (width 0.5) (layer F.Cu) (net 9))
 (segment (start 157.48 129.54) (end 160.02 132.08) (width 0.5) (layer B.Cu) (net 9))
 (segment (start 157.394966 147.32) (end 151.13 147.32) (width 0.5) (layer B.Cu) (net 9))
 (segment (start 160.02 144.694966) (end 157.394966 147.32) (width 0.5) (layer B.Cu) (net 9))
 (segment (start 160.02 132.08) (end 160.02 144.694966) (width 0.5) (layer B.Cu) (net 9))
 (segment (start 114.3 114.3) (end 116.84 111.76) (width 0.5) (layer F.Cu) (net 9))
 (segment (start 116.84 111.76) (end 146.05 111.76) (width 0.5) (layer F.Cu) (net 9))
 (segment (start 151.13 144.78) (end 157.48 144.78) (width 0.25) (layer B.Cu) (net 12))
 (segment (start 142.7225 116.3575) (end 142.24 116.84) (width 0.25) (layer F.Cu) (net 31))
 (segment (start 142.7225 114.3) (end 142.7225 116.3575) (width 0.25) (layer F.Cu) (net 31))
 (segment (start 109.22 114.3) (end 111.76 116.84) (width 0.25) (layer F.Cu) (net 8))
 (segment (start 123.19 113.03) (end 119.38 116.84) (width 0.25) (layer F.Cu) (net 8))
 (segment (start 124.9425 113.03) (end 123.19 113.03) (width 0.25) (layer F.Cu) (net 8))
 (segment (start 111.76 116.84) (end 119.38 116.84) (width 0.25) (layer F.Cu) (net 8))
 (segment (start 146.082024 136.26) (end 151.5 136.26) (width 0.25) (layer F.Cu) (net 4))
 (segment (start 154.94 139.7) (end 157.48 139.7) (width 0.25) (layer F.Cu) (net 4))
 (segment (start 151.5 136.26) (end 154.94 139.7) (width 0.25) (layer F.Cu) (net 4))
 (segment (start 160.02 149.86) (end 161.29 149.86) (width 0.25) (layer F.Cu) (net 4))
 (segment (start 161.29 149.86) (end 161.29 140.97) (width 0.25) (layer F.Cu) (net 4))
 (segment (start 160.02 139.7) (end 157.48 139.7) (width 0.25) (layer F.Cu) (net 4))
 (segment (start 161.29 140.97) (end 160.02 139.7) (width 0.25) (layer F.Cu) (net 4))
 (segment (start 106.68 134.62) (end 104.14 137.16) (width 0.25) (layer B.Cu) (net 4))
 (segment (start 111.76 134.62) (end 106.68 134.62) (width 0.25) (layer B.Cu) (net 4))
 (segment (start 119.38 127) (end 111.76 134.62) (width 0.25) (layer B.Cu) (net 4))
 (via (at 137.16 127) (size 0.8) (drill 0.4) (layers F.Cu B.Cu) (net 4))
 (segment (start 137.979989 127.819989) (end 146.05 135.89) (width 0.25) (layer F.Cu) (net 4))
 (segment (start 137.16 127) (end 137.979989 127.819989) (width 0.25) (layer F.Cu) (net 4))
 (segment (start 121.736421 128.256583) (end 121.736421 127.819989) (width 0.25) (layer F.Cu) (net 4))
 (segment (start 114.055 129.245) (end 120.748004 129.245) (width 0.25) (layer F.Cu) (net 4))
 (segment (start 120.748004 129.245) (end 121.736421 128.256583) (width 0.25) (layer F.Cu) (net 4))
 (via (at 121.92 126.365) (size 0.8) (drill 0.4) (layers F.Cu B.Cu) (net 4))
 (segment (start 121.736421 126.548579) (end 121.92 126.365) (width 0.25) (layer F.Cu) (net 4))
 (segment (start 121.736421 127.819989) (end 121.736421 126.548579) (width 0.25) (layer F.Cu) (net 4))
 (segment (start 121.92 126.365) (end 121.92 127) (width 0.25) (layer B.Cu) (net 4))
 (segment (start 121.92 127) (end 119.38 127) (width 0.25) (layer B.Cu) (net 4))
 (segment (start 137.16 127) (end 121.92 127) (width 0.25) (layer B.Cu) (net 4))
 (segment (start 146.082024 138.8) (end 151.5 138.8) (width 0.25) (layer F.Cu) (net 2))
 (segment (start 154.94 142.24) (end 157.48 142.24) (width 0.25) (layer F.Cu) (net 2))
 (segment (start 151.5 138.8) (end 154.94 142.24) (width 0.25) (layer F.Cu) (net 2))
 (segment (start 159.5375 147.32) (end 159.5375 143.0275) (width 0.25) (layer F.Cu) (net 2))
 (segment (start 158.75 142.24) (end 157.48 142.24) (width 0.25) (layer F.Cu) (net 2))
 (segment (start 159.5375 143.0275) (end 158.75 142.24) (width 0.25) (layer F.Cu) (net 2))
 (via (at 137.16 129.54) (size 0.8) (drill 0.4) (layers F.Cu B.Cu) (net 2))
 (segment (start 137.16 129.54) (end 138.43 130.81) (width 0.25) (layer F.Cu) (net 2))
 (segment (start 146.05 138.43) (end 138.43 130.81) (width 0.25) (layer F.Cu) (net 2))
 (segment (start 135.255 127.635) (end 137.16 129.54) (width 0.25) (layer B.Cu) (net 2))
 (segment (start 109.856411 137.16) (end 119.38141 127.635) (width 0.25) (layer B.Cu) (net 2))
 (segment (start 109.22 137.16) (end 109.856411 137.16) (width 0.25) (layer B.Cu) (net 2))
 (via (at 120.015 128.27) (size 0.8) (drill 0.4) (layers F.Cu B.Cu) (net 2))
 (segment (start 119.69 128.595) (end 120.015 128.27) (width 0.25) (layer F.Cu) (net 2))
 (segment (start 114.055 128.595) (end 119.69 128.595) (width 0.25) (layer F.Cu) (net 2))
 (segment (start 120.015 128.27) (end 120.015 127.635) (width 0.25) (layer B.Cu) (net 2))
 (segment (start 120.015 127.635) (end 135.255 127.635) (width 0.25) (layer B.Cu) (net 2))
 (segment (start 119.38141 127.635) (end 120.015 127.635) (width 0.25) (layer B.Cu) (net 2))
 (segment (start 101.965 150.13) (end 100.12 150.13) (width 0.25) (layer F.Cu) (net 18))
 (segment (start 102.6 150.13) (end 101.965 150.13) (width 0.25) (layer F.Cu) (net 18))
 (segment (start 113.93 138.8) (end 102.6 150.13) (width 0.25) (layer F.Cu) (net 18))
 (segment (start 123.222024 138.8) (end 113.93 138.8) (width 0.25) (layer F.Cu) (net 18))
 (segment (start 102.50641 152.13) (end 100.12 152.13) (width 0.25) (layer F.Cu) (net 20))
 (segment (start 123.222024 141.34) (end 113.29641 141.34) (width 0.25) (layer F.Cu) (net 20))
 (segment (start 113.29641 141.34) (end 102.50641 152.13) (width 0.25) (layer F.Cu) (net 20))
 (segment (start 123.222024 143.88) (end 122.197012 142.854988) (width 0.25) (layer F.Cu) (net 22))
 (segment (start 100.12 154.13) (end 102.41 154.13) (width 0.25) (layer F.Cu) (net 22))
 (segment (start 102.41 154.13) (end 113.685012 142.854988) (width 0.25) (layer F.Cu) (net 22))
 (segment (start 122.197012 142.854988) (end 113.685012 142.854988) (width 0.25) (layer F.Cu) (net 22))
 (segment (start 101.62 156.13) (end 100.12 156.13) (width 0.25) (layer F.Cu) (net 17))
 (segment (start 123.19 135.89) (end 117.475 135.89) (width 0.25) (layer B.Cu) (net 17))
 (segment (start 117.475 135.89) (end 114.935 138.43) (width 0.25) (layer B.Cu) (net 17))
 (via (at 114.935 145.415) (size 0.8) (drill 0.4) (layers F.Cu B.Cu) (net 17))
 (segment (start 114.935 138.43) (end 114.935 145.415) (width 0.25) (layer B.Cu) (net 17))
 (segment (start 112.395 145.415) (end 112.365 145.385) (width 0.25) (layer F.Cu) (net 17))
 (segment (start 112.365 145.385) (end 101.62 156.13) (width 0.25) (layer F.Cu) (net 17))
 (segment (start 114.935 145.415) (end 112.395 145.415) (width 0.25) (layer F.Cu) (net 17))
 (segment (start 116.205 124.46) (end 116.84 125.095) (width 0.25) (layer F.Cu) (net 10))
 (segment (start 116.84 125.095) (end 116.84 126.02) (width 0.25) (layer F.Cu) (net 10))
 (via (at 111.125 127) (size 0.8) (drill 0.4) (layers F.Cu B.Cu) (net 10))
 (segment (start 111.42 127.295) (end 111.125 127) (width 0.25) (layer F.Cu) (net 10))
 (segment (start 112.005 127.295) (end 111.42 127.295) (width 0.25) (layer F.Cu) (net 10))
 (segment (start 112.395 125.73) (end 114.3 125.73) (width 0.25) (layer B.Cu) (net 10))
 (via (at 114.3 125.73) (size 0.8) (drill 0.4) (layers F.Cu B.Cu) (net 10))
 (segment (start 111.125 127) (end 112.395 125.73) (width 0.25) (layer B.Cu) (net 10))
 (segment (start 114.3 125.73) (end 114.3 124.46) (width 0.25) (layer F.Cu) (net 10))
 (segment (start 114.3 124.46) (end 116.205 124.46) (width 0.25) (layer F.Cu) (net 10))
 (segment (start 113.8175 124.46) (end 114.3 124.46) (width 0.25) (layer F.Cu) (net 10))
 (segment (start 95.33 146.13) (end 95.25 146.05) (width 0.25) (layer F.Cu) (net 11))
 (segment (start 100.12 146.13) (end 95.33 146.13) (width 0.25) (layer F.Cu) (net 11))
 (segment (start 126.5175 115.57) (end 126.5175 113.03) (width 0.25) (layer F.Cu) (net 19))
 (segment (start 126.5175 115.57) (end 126.5175 122.7075) (width 0.25) (layer F.Cu) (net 19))
 (segment (start 126.5175 122.7075) (end 136.525 132.715) (width 0.25) (layer F.Cu) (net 19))
 (segment (start 136.525 132.715) (end 136.525 139.065) (width 0.25) (layer F.Cu) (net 19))
 (segment (start 138.43 140.97) (end 146.05 140.97) (width 0.25) (layer F.Cu) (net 19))
 (segment (start 136.525 139.065) (end 138.43 140.97) (width 0.25) (layer F.Cu) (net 19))
 (segment (start 123.19 146.05) (end 119.38 146.05) (width 0.25) (layer B.Cu) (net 23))
 (via (at 114.3 156.21) (size 0.8) (drill 0.4) (layers F.Cu B.Cu) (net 23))
 (segment (start 114.3 151.13) (end 114.3 156.21) (width 0.25) (layer B.Cu) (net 23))
 (segment (start 119.38 146.05) (end 114.3 151.13) (width 0.25) (layer B.Cu) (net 23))
 (segment (start 118.24 156.21) (end 118.32 156.13) (width 0.25) (layer F.Cu) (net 23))
 (segment (start 114.3 156.21) (end 118.24 156.21) (width 0.25) (layer F.Cu) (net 23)))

